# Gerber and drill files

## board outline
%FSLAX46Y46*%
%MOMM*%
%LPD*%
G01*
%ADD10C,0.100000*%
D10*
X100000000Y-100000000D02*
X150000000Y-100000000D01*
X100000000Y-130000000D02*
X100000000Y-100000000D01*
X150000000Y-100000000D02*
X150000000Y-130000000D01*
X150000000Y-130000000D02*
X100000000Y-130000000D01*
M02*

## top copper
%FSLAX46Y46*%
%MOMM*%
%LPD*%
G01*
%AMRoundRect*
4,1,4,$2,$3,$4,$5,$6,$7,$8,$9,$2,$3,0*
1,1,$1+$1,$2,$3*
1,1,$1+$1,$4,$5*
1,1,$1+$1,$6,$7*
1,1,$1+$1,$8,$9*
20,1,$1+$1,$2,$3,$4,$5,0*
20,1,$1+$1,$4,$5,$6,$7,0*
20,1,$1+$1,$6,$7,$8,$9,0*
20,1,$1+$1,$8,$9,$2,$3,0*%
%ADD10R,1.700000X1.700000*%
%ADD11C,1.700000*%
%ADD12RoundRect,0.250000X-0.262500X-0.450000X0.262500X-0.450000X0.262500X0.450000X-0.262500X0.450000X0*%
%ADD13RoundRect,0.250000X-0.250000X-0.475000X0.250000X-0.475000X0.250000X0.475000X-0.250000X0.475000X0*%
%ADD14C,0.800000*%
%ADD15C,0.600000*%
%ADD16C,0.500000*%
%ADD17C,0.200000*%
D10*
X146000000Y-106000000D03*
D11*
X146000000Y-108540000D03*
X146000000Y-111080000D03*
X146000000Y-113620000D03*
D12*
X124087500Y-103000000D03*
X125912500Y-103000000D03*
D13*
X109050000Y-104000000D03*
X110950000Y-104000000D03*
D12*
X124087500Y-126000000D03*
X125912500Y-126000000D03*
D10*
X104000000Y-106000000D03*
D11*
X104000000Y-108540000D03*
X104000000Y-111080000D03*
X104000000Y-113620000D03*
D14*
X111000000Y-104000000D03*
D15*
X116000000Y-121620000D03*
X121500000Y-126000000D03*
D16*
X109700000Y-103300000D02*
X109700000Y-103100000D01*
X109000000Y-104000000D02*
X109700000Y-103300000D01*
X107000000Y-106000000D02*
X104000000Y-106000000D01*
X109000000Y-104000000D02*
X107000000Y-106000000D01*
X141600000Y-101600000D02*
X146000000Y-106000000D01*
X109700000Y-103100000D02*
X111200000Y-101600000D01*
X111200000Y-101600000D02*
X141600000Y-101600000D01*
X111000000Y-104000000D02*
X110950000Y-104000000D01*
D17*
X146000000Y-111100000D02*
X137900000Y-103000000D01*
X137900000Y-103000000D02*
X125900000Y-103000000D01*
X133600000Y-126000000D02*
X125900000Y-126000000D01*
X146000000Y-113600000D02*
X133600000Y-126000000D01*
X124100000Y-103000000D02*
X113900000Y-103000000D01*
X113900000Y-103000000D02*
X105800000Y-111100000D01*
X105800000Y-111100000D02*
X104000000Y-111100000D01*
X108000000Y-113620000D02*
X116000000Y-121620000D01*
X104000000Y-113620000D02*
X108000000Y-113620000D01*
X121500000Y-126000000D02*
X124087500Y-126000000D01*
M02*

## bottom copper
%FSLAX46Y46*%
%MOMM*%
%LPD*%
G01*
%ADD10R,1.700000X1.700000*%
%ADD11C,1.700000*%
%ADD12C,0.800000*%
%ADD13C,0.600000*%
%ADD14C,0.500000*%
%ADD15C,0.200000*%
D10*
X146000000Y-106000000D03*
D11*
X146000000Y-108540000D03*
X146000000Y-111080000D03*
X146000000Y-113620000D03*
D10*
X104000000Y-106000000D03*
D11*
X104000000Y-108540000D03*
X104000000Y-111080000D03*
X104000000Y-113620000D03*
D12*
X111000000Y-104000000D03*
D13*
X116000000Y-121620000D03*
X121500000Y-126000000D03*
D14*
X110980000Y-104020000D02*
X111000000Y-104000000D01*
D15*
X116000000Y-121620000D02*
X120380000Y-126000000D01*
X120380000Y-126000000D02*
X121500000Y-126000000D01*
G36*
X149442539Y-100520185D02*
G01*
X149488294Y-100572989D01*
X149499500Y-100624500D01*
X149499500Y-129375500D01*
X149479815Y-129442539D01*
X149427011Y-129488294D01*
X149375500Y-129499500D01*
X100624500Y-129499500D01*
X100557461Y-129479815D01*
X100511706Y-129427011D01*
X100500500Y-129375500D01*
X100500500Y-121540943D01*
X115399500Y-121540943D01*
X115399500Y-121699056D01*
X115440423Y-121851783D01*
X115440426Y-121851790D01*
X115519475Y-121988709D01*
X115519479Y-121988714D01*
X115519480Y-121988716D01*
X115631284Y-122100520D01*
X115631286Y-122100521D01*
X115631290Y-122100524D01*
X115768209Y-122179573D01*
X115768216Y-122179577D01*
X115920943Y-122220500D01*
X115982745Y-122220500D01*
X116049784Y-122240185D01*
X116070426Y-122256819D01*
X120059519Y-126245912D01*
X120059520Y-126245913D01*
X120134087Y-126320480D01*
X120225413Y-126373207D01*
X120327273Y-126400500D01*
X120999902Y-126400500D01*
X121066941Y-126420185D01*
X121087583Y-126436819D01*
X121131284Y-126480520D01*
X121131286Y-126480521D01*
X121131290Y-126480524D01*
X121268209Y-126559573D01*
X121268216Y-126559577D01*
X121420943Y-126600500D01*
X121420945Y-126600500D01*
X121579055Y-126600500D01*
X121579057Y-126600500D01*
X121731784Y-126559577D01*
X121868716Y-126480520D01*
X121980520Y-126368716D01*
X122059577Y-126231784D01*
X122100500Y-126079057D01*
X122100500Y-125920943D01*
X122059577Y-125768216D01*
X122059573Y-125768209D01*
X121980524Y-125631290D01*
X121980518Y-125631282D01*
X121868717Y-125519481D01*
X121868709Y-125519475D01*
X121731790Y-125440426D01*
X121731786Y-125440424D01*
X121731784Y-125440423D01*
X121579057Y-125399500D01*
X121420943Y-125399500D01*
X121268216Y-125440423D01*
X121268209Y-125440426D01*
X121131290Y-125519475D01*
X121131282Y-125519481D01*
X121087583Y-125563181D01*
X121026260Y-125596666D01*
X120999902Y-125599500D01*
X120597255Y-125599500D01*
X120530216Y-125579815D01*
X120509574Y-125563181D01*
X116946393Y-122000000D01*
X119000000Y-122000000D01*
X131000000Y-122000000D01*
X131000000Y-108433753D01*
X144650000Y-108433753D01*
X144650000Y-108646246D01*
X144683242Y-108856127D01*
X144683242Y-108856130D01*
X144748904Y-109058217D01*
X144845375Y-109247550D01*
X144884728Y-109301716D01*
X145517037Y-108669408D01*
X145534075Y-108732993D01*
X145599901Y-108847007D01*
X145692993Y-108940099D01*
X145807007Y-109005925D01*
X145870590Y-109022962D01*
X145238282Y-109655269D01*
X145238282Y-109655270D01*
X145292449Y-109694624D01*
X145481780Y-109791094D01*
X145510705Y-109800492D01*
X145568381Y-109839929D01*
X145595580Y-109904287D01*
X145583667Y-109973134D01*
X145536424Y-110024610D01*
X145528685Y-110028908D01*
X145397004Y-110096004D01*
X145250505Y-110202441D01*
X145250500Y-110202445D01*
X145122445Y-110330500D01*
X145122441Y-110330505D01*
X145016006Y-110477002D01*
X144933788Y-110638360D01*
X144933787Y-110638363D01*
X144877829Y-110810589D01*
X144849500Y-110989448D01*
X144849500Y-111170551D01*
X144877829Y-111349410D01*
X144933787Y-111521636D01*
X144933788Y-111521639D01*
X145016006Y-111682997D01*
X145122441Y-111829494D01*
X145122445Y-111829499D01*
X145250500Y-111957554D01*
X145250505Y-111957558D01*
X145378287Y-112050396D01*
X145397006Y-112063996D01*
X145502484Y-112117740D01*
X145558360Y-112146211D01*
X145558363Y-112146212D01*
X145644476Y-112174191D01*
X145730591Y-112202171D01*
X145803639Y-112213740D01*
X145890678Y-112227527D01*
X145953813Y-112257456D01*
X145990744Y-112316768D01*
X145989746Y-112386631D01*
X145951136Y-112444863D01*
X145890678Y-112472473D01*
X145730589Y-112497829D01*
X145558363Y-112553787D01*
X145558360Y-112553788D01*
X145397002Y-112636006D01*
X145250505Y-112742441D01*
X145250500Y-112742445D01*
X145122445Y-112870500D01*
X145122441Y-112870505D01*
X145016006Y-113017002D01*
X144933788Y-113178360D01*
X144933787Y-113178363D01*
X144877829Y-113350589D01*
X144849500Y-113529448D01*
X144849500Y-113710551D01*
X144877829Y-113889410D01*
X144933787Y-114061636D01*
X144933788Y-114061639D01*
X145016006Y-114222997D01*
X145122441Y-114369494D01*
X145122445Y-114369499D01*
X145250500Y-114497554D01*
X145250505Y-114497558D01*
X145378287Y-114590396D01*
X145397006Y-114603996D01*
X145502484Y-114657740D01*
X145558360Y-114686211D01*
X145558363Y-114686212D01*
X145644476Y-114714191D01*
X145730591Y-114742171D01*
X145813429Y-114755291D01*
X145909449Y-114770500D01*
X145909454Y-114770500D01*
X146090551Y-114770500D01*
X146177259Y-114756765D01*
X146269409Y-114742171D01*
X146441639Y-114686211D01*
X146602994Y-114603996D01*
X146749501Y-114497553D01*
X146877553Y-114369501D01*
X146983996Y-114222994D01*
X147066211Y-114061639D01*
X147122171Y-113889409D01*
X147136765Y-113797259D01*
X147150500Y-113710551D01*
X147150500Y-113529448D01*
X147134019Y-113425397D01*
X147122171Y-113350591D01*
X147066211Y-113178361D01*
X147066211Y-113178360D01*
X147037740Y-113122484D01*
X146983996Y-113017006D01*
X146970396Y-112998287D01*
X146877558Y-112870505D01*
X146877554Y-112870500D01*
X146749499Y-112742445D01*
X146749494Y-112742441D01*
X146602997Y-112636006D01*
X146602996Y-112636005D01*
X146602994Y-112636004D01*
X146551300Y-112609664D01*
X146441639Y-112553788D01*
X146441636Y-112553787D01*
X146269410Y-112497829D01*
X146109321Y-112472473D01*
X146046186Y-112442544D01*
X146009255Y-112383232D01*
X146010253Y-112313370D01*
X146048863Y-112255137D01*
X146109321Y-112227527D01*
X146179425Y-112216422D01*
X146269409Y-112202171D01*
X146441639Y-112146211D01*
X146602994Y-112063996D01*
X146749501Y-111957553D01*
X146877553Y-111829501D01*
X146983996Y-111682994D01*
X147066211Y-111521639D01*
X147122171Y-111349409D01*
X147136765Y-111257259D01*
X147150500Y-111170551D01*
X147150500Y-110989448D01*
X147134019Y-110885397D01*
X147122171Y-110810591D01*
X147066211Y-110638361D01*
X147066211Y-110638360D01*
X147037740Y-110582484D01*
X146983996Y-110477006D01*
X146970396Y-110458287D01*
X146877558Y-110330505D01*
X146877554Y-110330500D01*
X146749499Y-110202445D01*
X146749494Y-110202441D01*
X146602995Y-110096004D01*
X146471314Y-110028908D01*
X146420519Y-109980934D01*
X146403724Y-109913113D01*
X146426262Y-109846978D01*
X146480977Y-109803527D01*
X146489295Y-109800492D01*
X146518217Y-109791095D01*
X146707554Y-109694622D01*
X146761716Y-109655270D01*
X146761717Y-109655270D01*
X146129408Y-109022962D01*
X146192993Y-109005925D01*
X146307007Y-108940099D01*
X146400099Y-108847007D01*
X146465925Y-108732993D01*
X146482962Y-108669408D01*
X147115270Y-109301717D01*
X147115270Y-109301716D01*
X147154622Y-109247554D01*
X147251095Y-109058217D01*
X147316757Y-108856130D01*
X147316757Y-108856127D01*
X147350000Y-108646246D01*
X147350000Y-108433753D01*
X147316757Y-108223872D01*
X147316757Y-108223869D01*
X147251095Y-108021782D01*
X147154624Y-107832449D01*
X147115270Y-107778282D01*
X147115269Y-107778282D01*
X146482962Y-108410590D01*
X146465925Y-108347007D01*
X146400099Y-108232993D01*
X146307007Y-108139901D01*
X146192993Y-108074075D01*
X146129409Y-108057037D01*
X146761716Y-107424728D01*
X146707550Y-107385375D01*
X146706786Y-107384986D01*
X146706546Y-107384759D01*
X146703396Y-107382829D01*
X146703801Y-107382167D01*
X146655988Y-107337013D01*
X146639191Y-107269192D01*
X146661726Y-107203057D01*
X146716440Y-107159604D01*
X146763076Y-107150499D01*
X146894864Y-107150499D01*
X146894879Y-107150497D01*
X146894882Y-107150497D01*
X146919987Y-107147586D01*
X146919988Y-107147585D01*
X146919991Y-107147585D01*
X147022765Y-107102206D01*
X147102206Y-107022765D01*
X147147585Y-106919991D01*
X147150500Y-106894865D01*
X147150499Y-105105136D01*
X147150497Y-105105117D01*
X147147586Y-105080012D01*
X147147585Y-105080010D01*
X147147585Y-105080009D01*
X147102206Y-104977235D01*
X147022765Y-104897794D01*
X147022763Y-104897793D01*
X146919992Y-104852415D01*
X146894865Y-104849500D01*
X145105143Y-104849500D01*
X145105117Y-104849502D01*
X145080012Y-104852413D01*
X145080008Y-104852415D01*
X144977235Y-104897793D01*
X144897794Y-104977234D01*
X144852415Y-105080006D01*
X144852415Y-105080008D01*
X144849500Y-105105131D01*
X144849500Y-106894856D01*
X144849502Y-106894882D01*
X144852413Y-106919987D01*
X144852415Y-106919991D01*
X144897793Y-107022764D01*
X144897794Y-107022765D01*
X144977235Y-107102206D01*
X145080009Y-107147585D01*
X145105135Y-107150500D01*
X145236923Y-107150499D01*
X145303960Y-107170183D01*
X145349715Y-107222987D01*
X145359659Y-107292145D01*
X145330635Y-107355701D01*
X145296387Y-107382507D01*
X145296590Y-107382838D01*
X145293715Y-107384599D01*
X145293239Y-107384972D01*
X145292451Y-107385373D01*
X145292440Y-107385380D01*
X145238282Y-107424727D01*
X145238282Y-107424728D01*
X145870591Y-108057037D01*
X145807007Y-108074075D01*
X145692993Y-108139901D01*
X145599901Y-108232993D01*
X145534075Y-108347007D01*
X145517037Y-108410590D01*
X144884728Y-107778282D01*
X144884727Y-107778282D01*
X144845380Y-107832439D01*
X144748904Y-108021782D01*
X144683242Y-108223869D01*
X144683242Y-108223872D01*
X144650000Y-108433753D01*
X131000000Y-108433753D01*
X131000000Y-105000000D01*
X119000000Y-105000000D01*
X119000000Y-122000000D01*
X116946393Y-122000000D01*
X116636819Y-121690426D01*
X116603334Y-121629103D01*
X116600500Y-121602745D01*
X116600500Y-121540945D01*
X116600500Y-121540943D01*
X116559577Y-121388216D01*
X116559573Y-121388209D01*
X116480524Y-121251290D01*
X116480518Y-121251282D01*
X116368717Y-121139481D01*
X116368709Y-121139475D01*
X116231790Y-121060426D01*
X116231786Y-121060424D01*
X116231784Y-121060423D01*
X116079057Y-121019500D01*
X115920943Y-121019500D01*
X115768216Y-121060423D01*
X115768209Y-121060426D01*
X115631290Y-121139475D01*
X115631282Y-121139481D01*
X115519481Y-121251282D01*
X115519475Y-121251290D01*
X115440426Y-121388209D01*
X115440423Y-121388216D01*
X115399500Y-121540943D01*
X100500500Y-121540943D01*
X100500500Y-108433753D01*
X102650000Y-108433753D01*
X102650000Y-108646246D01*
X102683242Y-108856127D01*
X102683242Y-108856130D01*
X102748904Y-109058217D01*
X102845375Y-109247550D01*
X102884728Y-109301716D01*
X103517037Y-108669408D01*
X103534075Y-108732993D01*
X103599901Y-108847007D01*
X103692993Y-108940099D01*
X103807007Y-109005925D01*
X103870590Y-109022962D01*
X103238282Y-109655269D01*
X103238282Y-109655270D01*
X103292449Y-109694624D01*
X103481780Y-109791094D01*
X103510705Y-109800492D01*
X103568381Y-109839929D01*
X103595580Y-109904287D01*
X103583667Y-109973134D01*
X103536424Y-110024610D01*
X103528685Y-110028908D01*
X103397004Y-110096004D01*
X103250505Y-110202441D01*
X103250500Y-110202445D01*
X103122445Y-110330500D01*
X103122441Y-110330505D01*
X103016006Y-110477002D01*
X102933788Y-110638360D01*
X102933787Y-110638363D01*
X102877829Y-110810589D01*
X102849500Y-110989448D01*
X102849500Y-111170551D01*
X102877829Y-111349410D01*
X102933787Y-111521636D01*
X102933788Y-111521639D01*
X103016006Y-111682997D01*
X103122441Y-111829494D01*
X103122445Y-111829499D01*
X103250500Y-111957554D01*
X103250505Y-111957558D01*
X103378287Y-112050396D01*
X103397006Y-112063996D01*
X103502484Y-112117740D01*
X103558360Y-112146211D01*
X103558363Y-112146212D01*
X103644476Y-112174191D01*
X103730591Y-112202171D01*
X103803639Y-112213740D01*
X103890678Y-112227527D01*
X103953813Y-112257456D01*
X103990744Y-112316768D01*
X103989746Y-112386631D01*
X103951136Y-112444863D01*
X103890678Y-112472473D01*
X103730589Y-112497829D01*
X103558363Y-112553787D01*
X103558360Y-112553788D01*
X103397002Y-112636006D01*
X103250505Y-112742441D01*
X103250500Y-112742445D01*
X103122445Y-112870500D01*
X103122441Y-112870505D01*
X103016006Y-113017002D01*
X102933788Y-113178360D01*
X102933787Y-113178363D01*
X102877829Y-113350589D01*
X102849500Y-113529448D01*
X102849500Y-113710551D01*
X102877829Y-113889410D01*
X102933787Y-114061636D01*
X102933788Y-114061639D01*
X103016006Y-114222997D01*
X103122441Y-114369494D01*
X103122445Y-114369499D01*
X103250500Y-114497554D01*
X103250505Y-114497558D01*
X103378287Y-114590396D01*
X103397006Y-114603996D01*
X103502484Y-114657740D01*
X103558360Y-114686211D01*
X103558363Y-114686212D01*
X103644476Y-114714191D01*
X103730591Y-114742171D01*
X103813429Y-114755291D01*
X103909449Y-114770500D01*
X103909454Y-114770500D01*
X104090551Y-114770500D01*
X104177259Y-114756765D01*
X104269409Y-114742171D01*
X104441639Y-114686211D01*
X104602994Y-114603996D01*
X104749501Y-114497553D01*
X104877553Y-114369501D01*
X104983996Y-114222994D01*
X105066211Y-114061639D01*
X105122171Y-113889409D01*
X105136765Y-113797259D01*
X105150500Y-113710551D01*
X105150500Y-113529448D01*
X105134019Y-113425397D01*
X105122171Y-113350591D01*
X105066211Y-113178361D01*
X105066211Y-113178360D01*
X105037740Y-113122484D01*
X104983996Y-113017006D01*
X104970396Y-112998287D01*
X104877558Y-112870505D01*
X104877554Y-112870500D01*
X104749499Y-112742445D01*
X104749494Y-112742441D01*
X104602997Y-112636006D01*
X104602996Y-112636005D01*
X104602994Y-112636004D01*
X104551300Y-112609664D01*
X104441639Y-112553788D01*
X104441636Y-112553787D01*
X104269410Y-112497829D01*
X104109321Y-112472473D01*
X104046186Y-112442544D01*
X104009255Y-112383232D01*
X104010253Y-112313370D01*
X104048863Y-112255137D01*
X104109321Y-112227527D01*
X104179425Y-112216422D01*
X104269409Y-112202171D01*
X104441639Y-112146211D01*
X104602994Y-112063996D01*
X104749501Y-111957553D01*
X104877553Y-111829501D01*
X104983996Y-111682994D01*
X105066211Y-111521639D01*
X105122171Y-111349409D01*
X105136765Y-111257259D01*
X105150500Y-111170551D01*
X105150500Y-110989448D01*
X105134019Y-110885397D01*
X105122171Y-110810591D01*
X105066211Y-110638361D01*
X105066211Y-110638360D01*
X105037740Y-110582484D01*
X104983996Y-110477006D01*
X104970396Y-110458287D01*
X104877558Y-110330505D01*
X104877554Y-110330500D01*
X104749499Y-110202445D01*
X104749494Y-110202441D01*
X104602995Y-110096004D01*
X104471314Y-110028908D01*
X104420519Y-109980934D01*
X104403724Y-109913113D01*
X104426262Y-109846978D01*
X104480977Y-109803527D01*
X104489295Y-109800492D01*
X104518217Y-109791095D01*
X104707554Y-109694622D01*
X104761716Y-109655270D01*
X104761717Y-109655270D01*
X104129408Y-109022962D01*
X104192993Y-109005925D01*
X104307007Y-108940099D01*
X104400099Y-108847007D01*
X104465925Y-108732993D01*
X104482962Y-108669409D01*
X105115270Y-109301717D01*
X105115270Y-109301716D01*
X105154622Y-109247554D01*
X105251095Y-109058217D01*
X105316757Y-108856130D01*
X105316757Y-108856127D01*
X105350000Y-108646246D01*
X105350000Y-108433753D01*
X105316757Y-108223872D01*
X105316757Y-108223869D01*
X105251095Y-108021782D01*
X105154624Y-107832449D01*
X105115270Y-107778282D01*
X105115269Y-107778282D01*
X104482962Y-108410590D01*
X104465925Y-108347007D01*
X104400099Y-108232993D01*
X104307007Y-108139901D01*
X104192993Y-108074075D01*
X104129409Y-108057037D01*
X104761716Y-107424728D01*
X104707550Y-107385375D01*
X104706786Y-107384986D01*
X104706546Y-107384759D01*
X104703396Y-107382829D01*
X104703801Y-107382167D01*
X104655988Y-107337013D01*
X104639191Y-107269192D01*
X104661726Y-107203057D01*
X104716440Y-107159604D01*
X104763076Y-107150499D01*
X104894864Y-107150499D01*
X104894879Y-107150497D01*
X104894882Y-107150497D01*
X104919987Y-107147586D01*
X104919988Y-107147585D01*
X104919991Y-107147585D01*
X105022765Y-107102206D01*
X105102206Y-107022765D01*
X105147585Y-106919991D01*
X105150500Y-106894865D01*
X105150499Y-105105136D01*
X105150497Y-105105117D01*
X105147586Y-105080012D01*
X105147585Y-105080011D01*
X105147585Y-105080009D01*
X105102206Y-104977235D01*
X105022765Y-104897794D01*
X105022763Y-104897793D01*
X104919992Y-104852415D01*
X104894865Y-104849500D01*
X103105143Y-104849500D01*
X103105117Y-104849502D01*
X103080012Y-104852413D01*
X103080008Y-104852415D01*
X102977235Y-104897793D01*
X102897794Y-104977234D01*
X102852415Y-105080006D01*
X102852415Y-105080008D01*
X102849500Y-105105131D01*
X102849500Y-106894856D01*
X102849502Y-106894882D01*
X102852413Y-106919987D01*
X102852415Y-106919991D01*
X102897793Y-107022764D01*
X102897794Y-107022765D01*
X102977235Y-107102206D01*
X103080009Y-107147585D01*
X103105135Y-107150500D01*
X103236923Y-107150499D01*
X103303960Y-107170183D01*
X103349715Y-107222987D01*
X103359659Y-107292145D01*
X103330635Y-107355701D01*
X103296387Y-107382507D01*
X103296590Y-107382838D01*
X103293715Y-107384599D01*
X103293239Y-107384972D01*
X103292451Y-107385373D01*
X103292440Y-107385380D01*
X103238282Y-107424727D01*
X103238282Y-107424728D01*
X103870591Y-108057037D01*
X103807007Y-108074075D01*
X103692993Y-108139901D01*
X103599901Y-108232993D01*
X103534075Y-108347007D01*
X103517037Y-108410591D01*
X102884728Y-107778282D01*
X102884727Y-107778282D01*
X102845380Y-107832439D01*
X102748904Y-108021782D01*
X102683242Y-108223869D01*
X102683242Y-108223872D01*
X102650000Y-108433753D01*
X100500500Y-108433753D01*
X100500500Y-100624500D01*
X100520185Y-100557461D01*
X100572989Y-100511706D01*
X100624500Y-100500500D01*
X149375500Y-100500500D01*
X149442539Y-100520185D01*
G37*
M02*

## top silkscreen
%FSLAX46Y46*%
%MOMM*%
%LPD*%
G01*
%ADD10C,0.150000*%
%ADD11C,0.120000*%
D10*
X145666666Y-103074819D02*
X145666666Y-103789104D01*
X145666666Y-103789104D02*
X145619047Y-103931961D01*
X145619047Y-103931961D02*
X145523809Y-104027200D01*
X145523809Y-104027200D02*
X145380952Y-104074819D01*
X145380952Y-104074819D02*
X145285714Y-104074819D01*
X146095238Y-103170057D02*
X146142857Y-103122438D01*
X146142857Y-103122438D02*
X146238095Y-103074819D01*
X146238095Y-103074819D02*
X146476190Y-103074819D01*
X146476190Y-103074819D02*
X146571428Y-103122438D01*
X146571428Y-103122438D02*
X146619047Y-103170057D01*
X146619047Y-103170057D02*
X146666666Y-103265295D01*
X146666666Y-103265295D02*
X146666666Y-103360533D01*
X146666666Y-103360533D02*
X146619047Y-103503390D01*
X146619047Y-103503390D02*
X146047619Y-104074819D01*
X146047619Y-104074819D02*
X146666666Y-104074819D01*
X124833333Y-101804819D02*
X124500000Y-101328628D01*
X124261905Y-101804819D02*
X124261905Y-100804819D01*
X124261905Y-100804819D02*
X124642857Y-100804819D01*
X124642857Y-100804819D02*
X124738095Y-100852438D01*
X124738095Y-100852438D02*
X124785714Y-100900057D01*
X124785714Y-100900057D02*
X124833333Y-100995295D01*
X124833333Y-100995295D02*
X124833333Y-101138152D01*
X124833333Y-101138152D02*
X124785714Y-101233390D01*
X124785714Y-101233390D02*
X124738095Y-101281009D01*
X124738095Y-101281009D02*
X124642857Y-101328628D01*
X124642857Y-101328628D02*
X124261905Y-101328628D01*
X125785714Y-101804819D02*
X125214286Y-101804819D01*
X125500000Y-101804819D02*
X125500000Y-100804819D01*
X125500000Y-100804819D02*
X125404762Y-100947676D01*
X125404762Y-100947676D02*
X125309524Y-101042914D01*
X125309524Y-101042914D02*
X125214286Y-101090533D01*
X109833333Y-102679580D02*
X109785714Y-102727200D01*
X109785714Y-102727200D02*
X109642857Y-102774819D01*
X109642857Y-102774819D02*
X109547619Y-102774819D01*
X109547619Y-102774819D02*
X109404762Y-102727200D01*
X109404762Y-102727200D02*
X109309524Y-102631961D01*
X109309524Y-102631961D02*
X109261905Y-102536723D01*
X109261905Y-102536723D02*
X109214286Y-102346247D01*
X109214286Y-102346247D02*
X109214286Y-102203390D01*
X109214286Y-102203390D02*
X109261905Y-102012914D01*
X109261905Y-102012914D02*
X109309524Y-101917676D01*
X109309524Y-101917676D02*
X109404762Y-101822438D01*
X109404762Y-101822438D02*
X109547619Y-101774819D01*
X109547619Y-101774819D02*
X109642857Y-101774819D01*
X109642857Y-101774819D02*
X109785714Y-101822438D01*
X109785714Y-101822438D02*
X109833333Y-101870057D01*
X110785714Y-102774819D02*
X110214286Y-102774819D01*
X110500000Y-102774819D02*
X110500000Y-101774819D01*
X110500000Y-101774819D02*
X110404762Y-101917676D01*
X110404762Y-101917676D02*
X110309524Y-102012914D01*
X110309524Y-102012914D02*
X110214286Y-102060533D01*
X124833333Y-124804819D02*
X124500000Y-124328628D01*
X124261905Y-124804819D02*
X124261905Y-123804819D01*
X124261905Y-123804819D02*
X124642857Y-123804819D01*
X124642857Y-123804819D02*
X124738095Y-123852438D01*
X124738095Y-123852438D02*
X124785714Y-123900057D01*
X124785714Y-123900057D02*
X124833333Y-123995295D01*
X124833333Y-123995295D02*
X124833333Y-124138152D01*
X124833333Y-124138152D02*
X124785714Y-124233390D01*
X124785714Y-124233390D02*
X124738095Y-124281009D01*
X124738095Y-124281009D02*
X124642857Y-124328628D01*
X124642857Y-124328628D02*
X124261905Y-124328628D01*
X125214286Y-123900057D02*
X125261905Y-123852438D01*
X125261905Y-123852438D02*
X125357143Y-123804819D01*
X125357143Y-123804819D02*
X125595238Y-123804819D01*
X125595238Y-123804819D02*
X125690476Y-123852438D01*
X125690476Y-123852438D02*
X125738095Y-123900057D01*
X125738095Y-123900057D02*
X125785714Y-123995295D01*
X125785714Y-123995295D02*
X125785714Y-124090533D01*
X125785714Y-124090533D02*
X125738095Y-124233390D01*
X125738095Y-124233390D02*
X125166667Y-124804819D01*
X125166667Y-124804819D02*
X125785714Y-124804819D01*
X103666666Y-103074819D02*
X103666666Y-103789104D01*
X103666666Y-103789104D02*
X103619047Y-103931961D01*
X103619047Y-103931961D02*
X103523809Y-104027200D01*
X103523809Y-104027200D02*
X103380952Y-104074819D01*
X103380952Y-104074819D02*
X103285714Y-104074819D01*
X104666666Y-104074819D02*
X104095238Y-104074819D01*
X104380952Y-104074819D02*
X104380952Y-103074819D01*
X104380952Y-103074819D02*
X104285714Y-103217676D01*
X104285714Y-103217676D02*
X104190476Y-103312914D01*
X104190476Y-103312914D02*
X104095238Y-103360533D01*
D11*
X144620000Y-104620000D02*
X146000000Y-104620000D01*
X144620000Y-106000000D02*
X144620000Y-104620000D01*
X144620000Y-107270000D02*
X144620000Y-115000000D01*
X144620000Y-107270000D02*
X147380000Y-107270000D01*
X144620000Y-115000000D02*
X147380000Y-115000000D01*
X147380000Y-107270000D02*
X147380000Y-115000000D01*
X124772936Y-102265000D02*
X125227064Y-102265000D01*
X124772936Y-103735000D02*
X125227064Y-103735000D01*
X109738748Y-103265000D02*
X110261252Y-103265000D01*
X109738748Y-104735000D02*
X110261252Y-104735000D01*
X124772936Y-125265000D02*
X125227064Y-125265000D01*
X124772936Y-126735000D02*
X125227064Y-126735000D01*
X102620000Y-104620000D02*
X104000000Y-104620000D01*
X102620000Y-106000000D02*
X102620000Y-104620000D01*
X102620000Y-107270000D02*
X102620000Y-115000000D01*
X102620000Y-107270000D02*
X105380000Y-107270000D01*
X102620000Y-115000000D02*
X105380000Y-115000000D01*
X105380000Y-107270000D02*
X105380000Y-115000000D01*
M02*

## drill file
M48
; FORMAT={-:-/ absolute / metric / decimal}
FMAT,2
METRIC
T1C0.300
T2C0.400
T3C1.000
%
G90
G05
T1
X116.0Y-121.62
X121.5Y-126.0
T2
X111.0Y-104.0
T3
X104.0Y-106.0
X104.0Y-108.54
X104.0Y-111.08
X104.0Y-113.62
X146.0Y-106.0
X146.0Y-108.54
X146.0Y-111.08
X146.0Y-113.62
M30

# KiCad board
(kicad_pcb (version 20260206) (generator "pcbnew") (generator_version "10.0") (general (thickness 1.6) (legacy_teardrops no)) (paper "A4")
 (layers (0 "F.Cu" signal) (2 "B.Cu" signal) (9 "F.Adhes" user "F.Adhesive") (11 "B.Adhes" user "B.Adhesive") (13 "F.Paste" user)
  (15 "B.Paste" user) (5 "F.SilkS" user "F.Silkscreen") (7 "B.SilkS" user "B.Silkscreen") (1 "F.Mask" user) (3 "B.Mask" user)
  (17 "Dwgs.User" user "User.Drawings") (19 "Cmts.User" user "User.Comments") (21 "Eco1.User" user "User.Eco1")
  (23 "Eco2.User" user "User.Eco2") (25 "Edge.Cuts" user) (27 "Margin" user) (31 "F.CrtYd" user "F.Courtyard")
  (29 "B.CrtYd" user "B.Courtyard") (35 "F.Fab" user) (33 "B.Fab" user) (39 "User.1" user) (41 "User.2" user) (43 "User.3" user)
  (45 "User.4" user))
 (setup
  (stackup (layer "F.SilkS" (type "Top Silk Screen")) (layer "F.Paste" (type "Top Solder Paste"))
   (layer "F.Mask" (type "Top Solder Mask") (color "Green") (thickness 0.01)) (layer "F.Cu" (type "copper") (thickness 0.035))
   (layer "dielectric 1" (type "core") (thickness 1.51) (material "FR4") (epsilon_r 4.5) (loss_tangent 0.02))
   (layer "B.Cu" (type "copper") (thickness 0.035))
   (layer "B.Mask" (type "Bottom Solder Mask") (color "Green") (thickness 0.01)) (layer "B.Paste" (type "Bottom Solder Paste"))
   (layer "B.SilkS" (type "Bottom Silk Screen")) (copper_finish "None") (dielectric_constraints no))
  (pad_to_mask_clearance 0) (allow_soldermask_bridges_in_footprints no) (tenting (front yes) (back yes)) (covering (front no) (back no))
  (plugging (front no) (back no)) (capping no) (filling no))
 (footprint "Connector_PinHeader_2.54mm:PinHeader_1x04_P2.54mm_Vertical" (layer "F.Cu") (at 146 106)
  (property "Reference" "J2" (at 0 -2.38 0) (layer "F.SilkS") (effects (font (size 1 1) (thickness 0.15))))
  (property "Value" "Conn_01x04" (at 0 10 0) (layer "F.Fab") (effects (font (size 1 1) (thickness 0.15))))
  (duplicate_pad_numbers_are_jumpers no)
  (fp_line (start -1.38 -1.38) (end 0 -1.38) (stroke (width 0.12) (type solid)) (layer "F.SilkS"))
  (fp_line (start -1.38 0) (end -1.38 -1.38) (stroke (width 0.12) (type solid)) (layer "F.SilkS"))
  (fp_line (start -1.38 1.27) (end -1.38 9) (stroke (width 0.12) (type solid)) (layer "F.SilkS"))
  (fp_line (start -1.38 1.27) (end 1.38 1.27) (stroke (width 0.12) (type solid)) (layer "F.SilkS"))
  (fp_line (start -1.38 9) (end 1.38 9) (stroke (width 0.12) (type solid)) (layer "F.SilkS"))
  (fp_line (start 1.38 1.27) (end 1.38 9) (stroke (width 0.12) (type solid)) (layer "F.SilkS"))
  (pad "1" thru_hole rect (at 0 0) (size 1.7 1.7) (drill 1) (layers "*.Cu" "*.Mask") (remove_unused_layers no) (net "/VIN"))
  (pad "2" thru_hole circle (at 0 2.54) (size 1.7 1.7) (drill 1) (layers "*.Cu" "*.Mask") (remove_unused_layers no) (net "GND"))
  (pad "3" thru_hole circle (at 0 5.08) (size 1.7 1.7) (drill 1) (layers "*.Cu" "*.Mask") (remove_unused_layers no) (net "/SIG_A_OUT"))
  (pad "4" thru_hole circle (at 0 7.62) (size 1.7 1.7) (drill 1) (layers "*.Cu" "*.Mask") (remove_unused_layers no) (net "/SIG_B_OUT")))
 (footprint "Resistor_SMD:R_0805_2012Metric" (layer "F.Cu") (at 125 103)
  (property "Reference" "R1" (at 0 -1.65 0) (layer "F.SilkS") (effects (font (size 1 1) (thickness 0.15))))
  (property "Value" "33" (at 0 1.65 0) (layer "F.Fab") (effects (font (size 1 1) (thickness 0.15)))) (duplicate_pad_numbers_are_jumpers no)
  (fp_line (start -0.227064 -0.735) (end 0.227064 -0.735) (stroke (width 0.12) (type solid)) (layer "F.SilkS"))
  (fp_line (start -0.227064 0.735) (end 0.227064 0.735) (stroke (width 0.12) (type solid)) (layer "F.SilkS"))
  (pad "1" smd roundrect (at -0.9125 0) (size 1.025 1.4) (layers "F.Cu" "F.Mask" "F.Paste") (roundrect_rratio 0.243902) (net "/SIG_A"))
  (pad "2" smd roundrect (at 0.9125 0) (size 1.025 1.4) (layers "F.Cu" "F.Mask" "F.Paste") (roundrect_rratio 0.243902) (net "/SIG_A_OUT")))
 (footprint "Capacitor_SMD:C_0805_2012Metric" (layer "F.Cu") (at 110 104)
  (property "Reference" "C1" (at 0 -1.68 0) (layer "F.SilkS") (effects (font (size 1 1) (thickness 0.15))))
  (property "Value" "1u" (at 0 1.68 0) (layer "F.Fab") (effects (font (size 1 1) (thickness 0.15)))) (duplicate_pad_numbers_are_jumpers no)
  (fp_line (start -0.261252 -0.735) (end 0.261252 -0.735) (stroke (width 0.12) (type solid)) (layer "F.SilkS"))
  (fp_line (start -0.261252 0.735) (end 0.261252 0.735) (stroke (width 0.12) (type solid)) (layer "F.SilkS"))
  (pad "1" smd roundrect (at -0.95 0) (size 1 1.45) (layers "F.Cu" "F.Mask" "F.Paste") (roundrect_rratio 0.25) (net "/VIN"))
  (pad "2" smd roundrect (at 0.95 0) (size 1 1.45) (layers "F.Cu" "F.Mask" "F.Paste") (roundrect_rratio 0.25) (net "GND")))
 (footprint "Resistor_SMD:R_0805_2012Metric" (layer "F.Cu") (at 125 126)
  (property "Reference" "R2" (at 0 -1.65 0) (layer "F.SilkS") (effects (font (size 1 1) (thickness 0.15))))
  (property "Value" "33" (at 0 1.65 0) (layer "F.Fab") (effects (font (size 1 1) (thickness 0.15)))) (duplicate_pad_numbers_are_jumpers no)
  (fp_line (start -0.227064 -0.735) (end 0.227064 -0.735) (stroke (width 0.12) (type solid)) (layer "F.SilkS"))
  (fp_line (start -0.227064 0.735) (end 0.227064 0.735) (stroke (width 0.12) (type solid)) (layer "F.SilkS"))
  (pad "1" smd roundrect (at -0.9125 0) (size 1.025 1.4) (layers "F.Cu" "F.Mask" "F.Paste") (roundrect_rratio 0.243902) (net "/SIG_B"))
  (pad "2" smd roundrect (at 0.9125 0) (size 1.025 1.4) (layers "F.Cu" "F.Mask" "F.Paste") (roundrect_rratio 0.243902) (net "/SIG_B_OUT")))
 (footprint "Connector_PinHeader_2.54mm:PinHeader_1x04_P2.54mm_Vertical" (layer "F.Cu") (at 104 106)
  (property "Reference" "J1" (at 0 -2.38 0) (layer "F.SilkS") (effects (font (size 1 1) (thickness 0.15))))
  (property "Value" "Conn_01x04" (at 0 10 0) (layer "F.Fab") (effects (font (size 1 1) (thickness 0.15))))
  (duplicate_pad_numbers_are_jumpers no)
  (fp_line (start -1.38 -1.38) (end 0 -1.38) (stroke (width 0.12) (type solid)) (layer "F.SilkS"))
  (fp_line (start -1.38 0) (end -1.38 -1.38) (stroke (width 0.12) (type solid)) (layer "F.SilkS"))
  (fp_line (start -1.38 1.27) (end -1.38 9) (stroke (width 0.12) (type solid)) (layer "F.SilkS"))
  (fp_line (start -1.38 1.27) (end 1.38 1.27) (stroke (width 0.12) (type solid)) (layer "F.SilkS"))
  (fp_line (start -1.38 9) (end 1.38 9) (stroke (width 0.12) (type solid)) (layer "F.SilkS"))
  (fp_line (start 1.38 1.27) (end 1.38 9) (stroke (width 0.12) (type solid)) (layer "F.SilkS"))
  (pad "1" thru_hole rect (at 0 0) (size 1.7 1.7) (drill 1) (layers "*.Cu" "*.Mask") (remove_unused_layers no) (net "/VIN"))
  (pad "2" thru_hole circle (at 0 2.54) (size 1.7 1.7) (drill 1) (layers "*.Cu" "*.Mask") (remove_unused_layers no) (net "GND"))
  (pad "3" thru_hole circle (at 0 5.08) (size 1.7 1.7) (drill 1) (layers "*.Cu" "*.Mask") (remove_unused_layers no) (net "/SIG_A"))
  (pad "4" thru_hole circle (at 0 7.62) (size 1.7 1.7) (drill 1) (layers "*.Cu" "*.Mask") (remove_unused_layers no) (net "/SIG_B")))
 (gr_line (start 100 100) (end 150 100) (stroke (width 0.1) (type default)) (layer "Edge.Cuts"))
 (gr_line (start 100 130) (end 100 100) (stroke (width 0.1) (type default)) (layer "Edge.Cuts"))
 (gr_line (start 150 100) (end 150 130) (stroke (width 0.1) (type default)) (layer "Edge.Cuts"))
 (gr_line (start 150 130) (end 100 130) (stroke (width 0.1) (type default)) (layer "Edge.Cuts"))
 (segment (start 109.7 103.3) (end 109.7 103.1) (width 0.5) (layer "F.Cu") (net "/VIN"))
 (segment (start 109 104) (end 109.7 103.3) (width 0.5) (layer "F.Cu") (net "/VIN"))
 (segment (start 107 106) (end 104 106) (width 0.5) (layer "F.Cu") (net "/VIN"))
 (segment (start 109 104) (end 107 106) (width 0.5) (layer "F.Cu") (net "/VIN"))
 (segment (start 141.6 101.6) (end 146 106) (width 0.5) (layer "F.Cu") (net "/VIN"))
 (segment (start 109.7 103.1) (end 111.2 101.6) (width 0.5) (layer "F.Cu") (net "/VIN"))
 (segment (start 111.2 101.6) (end 141.6 101.6) (width 0.5) (layer "F.Cu") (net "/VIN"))
 (segment (start 111 104) (end 110.95 104) (width 0.5) (layer "F.Cu") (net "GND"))
 (via (at 111 104) (size 0.8) (drill 0.4) (layers "F.Cu" "B.Cu") (capping yes) (filling yes) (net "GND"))
 (segment (start 110.98 104.02) (end 111 104) (width 0.5) (layer "B.Cu") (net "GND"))
 (segment (start 146 111.1) (end 137.9 103) (width 0.2) (layer "F.Cu") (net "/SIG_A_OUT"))
 (segment (start 137.9 103) (end 125.9 103) (width 0.2) (layer "F.Cu") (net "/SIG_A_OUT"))
 (segment (start 133.6 126) (end 125.9 126) (width 0.2) (layer "F.Cu") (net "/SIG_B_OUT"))
 (segment (start 146 113.6) (end 133.6 126) (width 0.2) (layer "F.Cu") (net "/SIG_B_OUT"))
 (segment (start 124.1 103) (end 113.9 103) (width 0.2) (layer "F.Cu") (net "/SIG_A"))
 (segment (start 113.9 103) (end 105.8 111.1) (width 0.2) (layer "F.Cu") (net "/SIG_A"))
 (segment (start 105.8 111.1) (end 104 111.1) (width 0.2) (layer "F.Cu") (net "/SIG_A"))
 (segment (start 108 113.62) (end 116 121.62) (width 0.2) (locked yes) (layer "F.Cu") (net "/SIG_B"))
 (segment (start 104 113.62) (end 108 113.62) (width 0.2) (locked yes) (layer "F.Cu") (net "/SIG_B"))
 (segment (start 121.5 126) (end 124.0875 126) (width 0.2) (locked yes) (layer "F.Cu") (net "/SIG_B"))
 (via (at 116 121.62) (size 0.6) (drill 0.3) (layers "F.Cu" "B.Cu") (locked yes) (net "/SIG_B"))
 (via (at 121.5 126) (size 0.6) (drill 0.3) (layers "F.Cu" "B.Cu") (locked yes) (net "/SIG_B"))
 (segment (start 116 121.62) (end 120.38 126) (width 0.2) (locked yes) (layer "B.Cu") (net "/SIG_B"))
 (segment (start 120.38 126) (end 121.5 126) (width 0.2) (locked yes) (layer "B.Cu") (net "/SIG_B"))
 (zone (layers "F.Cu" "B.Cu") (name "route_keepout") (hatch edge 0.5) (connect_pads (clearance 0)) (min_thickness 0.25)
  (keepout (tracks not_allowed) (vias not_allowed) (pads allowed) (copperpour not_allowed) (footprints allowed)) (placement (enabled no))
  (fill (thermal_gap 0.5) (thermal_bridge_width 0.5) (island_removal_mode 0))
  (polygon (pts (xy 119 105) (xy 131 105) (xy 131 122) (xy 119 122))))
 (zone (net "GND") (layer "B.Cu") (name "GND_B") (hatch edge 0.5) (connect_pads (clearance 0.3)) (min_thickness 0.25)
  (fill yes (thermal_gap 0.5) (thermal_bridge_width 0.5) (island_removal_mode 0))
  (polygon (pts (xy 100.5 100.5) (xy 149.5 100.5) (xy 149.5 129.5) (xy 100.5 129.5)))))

